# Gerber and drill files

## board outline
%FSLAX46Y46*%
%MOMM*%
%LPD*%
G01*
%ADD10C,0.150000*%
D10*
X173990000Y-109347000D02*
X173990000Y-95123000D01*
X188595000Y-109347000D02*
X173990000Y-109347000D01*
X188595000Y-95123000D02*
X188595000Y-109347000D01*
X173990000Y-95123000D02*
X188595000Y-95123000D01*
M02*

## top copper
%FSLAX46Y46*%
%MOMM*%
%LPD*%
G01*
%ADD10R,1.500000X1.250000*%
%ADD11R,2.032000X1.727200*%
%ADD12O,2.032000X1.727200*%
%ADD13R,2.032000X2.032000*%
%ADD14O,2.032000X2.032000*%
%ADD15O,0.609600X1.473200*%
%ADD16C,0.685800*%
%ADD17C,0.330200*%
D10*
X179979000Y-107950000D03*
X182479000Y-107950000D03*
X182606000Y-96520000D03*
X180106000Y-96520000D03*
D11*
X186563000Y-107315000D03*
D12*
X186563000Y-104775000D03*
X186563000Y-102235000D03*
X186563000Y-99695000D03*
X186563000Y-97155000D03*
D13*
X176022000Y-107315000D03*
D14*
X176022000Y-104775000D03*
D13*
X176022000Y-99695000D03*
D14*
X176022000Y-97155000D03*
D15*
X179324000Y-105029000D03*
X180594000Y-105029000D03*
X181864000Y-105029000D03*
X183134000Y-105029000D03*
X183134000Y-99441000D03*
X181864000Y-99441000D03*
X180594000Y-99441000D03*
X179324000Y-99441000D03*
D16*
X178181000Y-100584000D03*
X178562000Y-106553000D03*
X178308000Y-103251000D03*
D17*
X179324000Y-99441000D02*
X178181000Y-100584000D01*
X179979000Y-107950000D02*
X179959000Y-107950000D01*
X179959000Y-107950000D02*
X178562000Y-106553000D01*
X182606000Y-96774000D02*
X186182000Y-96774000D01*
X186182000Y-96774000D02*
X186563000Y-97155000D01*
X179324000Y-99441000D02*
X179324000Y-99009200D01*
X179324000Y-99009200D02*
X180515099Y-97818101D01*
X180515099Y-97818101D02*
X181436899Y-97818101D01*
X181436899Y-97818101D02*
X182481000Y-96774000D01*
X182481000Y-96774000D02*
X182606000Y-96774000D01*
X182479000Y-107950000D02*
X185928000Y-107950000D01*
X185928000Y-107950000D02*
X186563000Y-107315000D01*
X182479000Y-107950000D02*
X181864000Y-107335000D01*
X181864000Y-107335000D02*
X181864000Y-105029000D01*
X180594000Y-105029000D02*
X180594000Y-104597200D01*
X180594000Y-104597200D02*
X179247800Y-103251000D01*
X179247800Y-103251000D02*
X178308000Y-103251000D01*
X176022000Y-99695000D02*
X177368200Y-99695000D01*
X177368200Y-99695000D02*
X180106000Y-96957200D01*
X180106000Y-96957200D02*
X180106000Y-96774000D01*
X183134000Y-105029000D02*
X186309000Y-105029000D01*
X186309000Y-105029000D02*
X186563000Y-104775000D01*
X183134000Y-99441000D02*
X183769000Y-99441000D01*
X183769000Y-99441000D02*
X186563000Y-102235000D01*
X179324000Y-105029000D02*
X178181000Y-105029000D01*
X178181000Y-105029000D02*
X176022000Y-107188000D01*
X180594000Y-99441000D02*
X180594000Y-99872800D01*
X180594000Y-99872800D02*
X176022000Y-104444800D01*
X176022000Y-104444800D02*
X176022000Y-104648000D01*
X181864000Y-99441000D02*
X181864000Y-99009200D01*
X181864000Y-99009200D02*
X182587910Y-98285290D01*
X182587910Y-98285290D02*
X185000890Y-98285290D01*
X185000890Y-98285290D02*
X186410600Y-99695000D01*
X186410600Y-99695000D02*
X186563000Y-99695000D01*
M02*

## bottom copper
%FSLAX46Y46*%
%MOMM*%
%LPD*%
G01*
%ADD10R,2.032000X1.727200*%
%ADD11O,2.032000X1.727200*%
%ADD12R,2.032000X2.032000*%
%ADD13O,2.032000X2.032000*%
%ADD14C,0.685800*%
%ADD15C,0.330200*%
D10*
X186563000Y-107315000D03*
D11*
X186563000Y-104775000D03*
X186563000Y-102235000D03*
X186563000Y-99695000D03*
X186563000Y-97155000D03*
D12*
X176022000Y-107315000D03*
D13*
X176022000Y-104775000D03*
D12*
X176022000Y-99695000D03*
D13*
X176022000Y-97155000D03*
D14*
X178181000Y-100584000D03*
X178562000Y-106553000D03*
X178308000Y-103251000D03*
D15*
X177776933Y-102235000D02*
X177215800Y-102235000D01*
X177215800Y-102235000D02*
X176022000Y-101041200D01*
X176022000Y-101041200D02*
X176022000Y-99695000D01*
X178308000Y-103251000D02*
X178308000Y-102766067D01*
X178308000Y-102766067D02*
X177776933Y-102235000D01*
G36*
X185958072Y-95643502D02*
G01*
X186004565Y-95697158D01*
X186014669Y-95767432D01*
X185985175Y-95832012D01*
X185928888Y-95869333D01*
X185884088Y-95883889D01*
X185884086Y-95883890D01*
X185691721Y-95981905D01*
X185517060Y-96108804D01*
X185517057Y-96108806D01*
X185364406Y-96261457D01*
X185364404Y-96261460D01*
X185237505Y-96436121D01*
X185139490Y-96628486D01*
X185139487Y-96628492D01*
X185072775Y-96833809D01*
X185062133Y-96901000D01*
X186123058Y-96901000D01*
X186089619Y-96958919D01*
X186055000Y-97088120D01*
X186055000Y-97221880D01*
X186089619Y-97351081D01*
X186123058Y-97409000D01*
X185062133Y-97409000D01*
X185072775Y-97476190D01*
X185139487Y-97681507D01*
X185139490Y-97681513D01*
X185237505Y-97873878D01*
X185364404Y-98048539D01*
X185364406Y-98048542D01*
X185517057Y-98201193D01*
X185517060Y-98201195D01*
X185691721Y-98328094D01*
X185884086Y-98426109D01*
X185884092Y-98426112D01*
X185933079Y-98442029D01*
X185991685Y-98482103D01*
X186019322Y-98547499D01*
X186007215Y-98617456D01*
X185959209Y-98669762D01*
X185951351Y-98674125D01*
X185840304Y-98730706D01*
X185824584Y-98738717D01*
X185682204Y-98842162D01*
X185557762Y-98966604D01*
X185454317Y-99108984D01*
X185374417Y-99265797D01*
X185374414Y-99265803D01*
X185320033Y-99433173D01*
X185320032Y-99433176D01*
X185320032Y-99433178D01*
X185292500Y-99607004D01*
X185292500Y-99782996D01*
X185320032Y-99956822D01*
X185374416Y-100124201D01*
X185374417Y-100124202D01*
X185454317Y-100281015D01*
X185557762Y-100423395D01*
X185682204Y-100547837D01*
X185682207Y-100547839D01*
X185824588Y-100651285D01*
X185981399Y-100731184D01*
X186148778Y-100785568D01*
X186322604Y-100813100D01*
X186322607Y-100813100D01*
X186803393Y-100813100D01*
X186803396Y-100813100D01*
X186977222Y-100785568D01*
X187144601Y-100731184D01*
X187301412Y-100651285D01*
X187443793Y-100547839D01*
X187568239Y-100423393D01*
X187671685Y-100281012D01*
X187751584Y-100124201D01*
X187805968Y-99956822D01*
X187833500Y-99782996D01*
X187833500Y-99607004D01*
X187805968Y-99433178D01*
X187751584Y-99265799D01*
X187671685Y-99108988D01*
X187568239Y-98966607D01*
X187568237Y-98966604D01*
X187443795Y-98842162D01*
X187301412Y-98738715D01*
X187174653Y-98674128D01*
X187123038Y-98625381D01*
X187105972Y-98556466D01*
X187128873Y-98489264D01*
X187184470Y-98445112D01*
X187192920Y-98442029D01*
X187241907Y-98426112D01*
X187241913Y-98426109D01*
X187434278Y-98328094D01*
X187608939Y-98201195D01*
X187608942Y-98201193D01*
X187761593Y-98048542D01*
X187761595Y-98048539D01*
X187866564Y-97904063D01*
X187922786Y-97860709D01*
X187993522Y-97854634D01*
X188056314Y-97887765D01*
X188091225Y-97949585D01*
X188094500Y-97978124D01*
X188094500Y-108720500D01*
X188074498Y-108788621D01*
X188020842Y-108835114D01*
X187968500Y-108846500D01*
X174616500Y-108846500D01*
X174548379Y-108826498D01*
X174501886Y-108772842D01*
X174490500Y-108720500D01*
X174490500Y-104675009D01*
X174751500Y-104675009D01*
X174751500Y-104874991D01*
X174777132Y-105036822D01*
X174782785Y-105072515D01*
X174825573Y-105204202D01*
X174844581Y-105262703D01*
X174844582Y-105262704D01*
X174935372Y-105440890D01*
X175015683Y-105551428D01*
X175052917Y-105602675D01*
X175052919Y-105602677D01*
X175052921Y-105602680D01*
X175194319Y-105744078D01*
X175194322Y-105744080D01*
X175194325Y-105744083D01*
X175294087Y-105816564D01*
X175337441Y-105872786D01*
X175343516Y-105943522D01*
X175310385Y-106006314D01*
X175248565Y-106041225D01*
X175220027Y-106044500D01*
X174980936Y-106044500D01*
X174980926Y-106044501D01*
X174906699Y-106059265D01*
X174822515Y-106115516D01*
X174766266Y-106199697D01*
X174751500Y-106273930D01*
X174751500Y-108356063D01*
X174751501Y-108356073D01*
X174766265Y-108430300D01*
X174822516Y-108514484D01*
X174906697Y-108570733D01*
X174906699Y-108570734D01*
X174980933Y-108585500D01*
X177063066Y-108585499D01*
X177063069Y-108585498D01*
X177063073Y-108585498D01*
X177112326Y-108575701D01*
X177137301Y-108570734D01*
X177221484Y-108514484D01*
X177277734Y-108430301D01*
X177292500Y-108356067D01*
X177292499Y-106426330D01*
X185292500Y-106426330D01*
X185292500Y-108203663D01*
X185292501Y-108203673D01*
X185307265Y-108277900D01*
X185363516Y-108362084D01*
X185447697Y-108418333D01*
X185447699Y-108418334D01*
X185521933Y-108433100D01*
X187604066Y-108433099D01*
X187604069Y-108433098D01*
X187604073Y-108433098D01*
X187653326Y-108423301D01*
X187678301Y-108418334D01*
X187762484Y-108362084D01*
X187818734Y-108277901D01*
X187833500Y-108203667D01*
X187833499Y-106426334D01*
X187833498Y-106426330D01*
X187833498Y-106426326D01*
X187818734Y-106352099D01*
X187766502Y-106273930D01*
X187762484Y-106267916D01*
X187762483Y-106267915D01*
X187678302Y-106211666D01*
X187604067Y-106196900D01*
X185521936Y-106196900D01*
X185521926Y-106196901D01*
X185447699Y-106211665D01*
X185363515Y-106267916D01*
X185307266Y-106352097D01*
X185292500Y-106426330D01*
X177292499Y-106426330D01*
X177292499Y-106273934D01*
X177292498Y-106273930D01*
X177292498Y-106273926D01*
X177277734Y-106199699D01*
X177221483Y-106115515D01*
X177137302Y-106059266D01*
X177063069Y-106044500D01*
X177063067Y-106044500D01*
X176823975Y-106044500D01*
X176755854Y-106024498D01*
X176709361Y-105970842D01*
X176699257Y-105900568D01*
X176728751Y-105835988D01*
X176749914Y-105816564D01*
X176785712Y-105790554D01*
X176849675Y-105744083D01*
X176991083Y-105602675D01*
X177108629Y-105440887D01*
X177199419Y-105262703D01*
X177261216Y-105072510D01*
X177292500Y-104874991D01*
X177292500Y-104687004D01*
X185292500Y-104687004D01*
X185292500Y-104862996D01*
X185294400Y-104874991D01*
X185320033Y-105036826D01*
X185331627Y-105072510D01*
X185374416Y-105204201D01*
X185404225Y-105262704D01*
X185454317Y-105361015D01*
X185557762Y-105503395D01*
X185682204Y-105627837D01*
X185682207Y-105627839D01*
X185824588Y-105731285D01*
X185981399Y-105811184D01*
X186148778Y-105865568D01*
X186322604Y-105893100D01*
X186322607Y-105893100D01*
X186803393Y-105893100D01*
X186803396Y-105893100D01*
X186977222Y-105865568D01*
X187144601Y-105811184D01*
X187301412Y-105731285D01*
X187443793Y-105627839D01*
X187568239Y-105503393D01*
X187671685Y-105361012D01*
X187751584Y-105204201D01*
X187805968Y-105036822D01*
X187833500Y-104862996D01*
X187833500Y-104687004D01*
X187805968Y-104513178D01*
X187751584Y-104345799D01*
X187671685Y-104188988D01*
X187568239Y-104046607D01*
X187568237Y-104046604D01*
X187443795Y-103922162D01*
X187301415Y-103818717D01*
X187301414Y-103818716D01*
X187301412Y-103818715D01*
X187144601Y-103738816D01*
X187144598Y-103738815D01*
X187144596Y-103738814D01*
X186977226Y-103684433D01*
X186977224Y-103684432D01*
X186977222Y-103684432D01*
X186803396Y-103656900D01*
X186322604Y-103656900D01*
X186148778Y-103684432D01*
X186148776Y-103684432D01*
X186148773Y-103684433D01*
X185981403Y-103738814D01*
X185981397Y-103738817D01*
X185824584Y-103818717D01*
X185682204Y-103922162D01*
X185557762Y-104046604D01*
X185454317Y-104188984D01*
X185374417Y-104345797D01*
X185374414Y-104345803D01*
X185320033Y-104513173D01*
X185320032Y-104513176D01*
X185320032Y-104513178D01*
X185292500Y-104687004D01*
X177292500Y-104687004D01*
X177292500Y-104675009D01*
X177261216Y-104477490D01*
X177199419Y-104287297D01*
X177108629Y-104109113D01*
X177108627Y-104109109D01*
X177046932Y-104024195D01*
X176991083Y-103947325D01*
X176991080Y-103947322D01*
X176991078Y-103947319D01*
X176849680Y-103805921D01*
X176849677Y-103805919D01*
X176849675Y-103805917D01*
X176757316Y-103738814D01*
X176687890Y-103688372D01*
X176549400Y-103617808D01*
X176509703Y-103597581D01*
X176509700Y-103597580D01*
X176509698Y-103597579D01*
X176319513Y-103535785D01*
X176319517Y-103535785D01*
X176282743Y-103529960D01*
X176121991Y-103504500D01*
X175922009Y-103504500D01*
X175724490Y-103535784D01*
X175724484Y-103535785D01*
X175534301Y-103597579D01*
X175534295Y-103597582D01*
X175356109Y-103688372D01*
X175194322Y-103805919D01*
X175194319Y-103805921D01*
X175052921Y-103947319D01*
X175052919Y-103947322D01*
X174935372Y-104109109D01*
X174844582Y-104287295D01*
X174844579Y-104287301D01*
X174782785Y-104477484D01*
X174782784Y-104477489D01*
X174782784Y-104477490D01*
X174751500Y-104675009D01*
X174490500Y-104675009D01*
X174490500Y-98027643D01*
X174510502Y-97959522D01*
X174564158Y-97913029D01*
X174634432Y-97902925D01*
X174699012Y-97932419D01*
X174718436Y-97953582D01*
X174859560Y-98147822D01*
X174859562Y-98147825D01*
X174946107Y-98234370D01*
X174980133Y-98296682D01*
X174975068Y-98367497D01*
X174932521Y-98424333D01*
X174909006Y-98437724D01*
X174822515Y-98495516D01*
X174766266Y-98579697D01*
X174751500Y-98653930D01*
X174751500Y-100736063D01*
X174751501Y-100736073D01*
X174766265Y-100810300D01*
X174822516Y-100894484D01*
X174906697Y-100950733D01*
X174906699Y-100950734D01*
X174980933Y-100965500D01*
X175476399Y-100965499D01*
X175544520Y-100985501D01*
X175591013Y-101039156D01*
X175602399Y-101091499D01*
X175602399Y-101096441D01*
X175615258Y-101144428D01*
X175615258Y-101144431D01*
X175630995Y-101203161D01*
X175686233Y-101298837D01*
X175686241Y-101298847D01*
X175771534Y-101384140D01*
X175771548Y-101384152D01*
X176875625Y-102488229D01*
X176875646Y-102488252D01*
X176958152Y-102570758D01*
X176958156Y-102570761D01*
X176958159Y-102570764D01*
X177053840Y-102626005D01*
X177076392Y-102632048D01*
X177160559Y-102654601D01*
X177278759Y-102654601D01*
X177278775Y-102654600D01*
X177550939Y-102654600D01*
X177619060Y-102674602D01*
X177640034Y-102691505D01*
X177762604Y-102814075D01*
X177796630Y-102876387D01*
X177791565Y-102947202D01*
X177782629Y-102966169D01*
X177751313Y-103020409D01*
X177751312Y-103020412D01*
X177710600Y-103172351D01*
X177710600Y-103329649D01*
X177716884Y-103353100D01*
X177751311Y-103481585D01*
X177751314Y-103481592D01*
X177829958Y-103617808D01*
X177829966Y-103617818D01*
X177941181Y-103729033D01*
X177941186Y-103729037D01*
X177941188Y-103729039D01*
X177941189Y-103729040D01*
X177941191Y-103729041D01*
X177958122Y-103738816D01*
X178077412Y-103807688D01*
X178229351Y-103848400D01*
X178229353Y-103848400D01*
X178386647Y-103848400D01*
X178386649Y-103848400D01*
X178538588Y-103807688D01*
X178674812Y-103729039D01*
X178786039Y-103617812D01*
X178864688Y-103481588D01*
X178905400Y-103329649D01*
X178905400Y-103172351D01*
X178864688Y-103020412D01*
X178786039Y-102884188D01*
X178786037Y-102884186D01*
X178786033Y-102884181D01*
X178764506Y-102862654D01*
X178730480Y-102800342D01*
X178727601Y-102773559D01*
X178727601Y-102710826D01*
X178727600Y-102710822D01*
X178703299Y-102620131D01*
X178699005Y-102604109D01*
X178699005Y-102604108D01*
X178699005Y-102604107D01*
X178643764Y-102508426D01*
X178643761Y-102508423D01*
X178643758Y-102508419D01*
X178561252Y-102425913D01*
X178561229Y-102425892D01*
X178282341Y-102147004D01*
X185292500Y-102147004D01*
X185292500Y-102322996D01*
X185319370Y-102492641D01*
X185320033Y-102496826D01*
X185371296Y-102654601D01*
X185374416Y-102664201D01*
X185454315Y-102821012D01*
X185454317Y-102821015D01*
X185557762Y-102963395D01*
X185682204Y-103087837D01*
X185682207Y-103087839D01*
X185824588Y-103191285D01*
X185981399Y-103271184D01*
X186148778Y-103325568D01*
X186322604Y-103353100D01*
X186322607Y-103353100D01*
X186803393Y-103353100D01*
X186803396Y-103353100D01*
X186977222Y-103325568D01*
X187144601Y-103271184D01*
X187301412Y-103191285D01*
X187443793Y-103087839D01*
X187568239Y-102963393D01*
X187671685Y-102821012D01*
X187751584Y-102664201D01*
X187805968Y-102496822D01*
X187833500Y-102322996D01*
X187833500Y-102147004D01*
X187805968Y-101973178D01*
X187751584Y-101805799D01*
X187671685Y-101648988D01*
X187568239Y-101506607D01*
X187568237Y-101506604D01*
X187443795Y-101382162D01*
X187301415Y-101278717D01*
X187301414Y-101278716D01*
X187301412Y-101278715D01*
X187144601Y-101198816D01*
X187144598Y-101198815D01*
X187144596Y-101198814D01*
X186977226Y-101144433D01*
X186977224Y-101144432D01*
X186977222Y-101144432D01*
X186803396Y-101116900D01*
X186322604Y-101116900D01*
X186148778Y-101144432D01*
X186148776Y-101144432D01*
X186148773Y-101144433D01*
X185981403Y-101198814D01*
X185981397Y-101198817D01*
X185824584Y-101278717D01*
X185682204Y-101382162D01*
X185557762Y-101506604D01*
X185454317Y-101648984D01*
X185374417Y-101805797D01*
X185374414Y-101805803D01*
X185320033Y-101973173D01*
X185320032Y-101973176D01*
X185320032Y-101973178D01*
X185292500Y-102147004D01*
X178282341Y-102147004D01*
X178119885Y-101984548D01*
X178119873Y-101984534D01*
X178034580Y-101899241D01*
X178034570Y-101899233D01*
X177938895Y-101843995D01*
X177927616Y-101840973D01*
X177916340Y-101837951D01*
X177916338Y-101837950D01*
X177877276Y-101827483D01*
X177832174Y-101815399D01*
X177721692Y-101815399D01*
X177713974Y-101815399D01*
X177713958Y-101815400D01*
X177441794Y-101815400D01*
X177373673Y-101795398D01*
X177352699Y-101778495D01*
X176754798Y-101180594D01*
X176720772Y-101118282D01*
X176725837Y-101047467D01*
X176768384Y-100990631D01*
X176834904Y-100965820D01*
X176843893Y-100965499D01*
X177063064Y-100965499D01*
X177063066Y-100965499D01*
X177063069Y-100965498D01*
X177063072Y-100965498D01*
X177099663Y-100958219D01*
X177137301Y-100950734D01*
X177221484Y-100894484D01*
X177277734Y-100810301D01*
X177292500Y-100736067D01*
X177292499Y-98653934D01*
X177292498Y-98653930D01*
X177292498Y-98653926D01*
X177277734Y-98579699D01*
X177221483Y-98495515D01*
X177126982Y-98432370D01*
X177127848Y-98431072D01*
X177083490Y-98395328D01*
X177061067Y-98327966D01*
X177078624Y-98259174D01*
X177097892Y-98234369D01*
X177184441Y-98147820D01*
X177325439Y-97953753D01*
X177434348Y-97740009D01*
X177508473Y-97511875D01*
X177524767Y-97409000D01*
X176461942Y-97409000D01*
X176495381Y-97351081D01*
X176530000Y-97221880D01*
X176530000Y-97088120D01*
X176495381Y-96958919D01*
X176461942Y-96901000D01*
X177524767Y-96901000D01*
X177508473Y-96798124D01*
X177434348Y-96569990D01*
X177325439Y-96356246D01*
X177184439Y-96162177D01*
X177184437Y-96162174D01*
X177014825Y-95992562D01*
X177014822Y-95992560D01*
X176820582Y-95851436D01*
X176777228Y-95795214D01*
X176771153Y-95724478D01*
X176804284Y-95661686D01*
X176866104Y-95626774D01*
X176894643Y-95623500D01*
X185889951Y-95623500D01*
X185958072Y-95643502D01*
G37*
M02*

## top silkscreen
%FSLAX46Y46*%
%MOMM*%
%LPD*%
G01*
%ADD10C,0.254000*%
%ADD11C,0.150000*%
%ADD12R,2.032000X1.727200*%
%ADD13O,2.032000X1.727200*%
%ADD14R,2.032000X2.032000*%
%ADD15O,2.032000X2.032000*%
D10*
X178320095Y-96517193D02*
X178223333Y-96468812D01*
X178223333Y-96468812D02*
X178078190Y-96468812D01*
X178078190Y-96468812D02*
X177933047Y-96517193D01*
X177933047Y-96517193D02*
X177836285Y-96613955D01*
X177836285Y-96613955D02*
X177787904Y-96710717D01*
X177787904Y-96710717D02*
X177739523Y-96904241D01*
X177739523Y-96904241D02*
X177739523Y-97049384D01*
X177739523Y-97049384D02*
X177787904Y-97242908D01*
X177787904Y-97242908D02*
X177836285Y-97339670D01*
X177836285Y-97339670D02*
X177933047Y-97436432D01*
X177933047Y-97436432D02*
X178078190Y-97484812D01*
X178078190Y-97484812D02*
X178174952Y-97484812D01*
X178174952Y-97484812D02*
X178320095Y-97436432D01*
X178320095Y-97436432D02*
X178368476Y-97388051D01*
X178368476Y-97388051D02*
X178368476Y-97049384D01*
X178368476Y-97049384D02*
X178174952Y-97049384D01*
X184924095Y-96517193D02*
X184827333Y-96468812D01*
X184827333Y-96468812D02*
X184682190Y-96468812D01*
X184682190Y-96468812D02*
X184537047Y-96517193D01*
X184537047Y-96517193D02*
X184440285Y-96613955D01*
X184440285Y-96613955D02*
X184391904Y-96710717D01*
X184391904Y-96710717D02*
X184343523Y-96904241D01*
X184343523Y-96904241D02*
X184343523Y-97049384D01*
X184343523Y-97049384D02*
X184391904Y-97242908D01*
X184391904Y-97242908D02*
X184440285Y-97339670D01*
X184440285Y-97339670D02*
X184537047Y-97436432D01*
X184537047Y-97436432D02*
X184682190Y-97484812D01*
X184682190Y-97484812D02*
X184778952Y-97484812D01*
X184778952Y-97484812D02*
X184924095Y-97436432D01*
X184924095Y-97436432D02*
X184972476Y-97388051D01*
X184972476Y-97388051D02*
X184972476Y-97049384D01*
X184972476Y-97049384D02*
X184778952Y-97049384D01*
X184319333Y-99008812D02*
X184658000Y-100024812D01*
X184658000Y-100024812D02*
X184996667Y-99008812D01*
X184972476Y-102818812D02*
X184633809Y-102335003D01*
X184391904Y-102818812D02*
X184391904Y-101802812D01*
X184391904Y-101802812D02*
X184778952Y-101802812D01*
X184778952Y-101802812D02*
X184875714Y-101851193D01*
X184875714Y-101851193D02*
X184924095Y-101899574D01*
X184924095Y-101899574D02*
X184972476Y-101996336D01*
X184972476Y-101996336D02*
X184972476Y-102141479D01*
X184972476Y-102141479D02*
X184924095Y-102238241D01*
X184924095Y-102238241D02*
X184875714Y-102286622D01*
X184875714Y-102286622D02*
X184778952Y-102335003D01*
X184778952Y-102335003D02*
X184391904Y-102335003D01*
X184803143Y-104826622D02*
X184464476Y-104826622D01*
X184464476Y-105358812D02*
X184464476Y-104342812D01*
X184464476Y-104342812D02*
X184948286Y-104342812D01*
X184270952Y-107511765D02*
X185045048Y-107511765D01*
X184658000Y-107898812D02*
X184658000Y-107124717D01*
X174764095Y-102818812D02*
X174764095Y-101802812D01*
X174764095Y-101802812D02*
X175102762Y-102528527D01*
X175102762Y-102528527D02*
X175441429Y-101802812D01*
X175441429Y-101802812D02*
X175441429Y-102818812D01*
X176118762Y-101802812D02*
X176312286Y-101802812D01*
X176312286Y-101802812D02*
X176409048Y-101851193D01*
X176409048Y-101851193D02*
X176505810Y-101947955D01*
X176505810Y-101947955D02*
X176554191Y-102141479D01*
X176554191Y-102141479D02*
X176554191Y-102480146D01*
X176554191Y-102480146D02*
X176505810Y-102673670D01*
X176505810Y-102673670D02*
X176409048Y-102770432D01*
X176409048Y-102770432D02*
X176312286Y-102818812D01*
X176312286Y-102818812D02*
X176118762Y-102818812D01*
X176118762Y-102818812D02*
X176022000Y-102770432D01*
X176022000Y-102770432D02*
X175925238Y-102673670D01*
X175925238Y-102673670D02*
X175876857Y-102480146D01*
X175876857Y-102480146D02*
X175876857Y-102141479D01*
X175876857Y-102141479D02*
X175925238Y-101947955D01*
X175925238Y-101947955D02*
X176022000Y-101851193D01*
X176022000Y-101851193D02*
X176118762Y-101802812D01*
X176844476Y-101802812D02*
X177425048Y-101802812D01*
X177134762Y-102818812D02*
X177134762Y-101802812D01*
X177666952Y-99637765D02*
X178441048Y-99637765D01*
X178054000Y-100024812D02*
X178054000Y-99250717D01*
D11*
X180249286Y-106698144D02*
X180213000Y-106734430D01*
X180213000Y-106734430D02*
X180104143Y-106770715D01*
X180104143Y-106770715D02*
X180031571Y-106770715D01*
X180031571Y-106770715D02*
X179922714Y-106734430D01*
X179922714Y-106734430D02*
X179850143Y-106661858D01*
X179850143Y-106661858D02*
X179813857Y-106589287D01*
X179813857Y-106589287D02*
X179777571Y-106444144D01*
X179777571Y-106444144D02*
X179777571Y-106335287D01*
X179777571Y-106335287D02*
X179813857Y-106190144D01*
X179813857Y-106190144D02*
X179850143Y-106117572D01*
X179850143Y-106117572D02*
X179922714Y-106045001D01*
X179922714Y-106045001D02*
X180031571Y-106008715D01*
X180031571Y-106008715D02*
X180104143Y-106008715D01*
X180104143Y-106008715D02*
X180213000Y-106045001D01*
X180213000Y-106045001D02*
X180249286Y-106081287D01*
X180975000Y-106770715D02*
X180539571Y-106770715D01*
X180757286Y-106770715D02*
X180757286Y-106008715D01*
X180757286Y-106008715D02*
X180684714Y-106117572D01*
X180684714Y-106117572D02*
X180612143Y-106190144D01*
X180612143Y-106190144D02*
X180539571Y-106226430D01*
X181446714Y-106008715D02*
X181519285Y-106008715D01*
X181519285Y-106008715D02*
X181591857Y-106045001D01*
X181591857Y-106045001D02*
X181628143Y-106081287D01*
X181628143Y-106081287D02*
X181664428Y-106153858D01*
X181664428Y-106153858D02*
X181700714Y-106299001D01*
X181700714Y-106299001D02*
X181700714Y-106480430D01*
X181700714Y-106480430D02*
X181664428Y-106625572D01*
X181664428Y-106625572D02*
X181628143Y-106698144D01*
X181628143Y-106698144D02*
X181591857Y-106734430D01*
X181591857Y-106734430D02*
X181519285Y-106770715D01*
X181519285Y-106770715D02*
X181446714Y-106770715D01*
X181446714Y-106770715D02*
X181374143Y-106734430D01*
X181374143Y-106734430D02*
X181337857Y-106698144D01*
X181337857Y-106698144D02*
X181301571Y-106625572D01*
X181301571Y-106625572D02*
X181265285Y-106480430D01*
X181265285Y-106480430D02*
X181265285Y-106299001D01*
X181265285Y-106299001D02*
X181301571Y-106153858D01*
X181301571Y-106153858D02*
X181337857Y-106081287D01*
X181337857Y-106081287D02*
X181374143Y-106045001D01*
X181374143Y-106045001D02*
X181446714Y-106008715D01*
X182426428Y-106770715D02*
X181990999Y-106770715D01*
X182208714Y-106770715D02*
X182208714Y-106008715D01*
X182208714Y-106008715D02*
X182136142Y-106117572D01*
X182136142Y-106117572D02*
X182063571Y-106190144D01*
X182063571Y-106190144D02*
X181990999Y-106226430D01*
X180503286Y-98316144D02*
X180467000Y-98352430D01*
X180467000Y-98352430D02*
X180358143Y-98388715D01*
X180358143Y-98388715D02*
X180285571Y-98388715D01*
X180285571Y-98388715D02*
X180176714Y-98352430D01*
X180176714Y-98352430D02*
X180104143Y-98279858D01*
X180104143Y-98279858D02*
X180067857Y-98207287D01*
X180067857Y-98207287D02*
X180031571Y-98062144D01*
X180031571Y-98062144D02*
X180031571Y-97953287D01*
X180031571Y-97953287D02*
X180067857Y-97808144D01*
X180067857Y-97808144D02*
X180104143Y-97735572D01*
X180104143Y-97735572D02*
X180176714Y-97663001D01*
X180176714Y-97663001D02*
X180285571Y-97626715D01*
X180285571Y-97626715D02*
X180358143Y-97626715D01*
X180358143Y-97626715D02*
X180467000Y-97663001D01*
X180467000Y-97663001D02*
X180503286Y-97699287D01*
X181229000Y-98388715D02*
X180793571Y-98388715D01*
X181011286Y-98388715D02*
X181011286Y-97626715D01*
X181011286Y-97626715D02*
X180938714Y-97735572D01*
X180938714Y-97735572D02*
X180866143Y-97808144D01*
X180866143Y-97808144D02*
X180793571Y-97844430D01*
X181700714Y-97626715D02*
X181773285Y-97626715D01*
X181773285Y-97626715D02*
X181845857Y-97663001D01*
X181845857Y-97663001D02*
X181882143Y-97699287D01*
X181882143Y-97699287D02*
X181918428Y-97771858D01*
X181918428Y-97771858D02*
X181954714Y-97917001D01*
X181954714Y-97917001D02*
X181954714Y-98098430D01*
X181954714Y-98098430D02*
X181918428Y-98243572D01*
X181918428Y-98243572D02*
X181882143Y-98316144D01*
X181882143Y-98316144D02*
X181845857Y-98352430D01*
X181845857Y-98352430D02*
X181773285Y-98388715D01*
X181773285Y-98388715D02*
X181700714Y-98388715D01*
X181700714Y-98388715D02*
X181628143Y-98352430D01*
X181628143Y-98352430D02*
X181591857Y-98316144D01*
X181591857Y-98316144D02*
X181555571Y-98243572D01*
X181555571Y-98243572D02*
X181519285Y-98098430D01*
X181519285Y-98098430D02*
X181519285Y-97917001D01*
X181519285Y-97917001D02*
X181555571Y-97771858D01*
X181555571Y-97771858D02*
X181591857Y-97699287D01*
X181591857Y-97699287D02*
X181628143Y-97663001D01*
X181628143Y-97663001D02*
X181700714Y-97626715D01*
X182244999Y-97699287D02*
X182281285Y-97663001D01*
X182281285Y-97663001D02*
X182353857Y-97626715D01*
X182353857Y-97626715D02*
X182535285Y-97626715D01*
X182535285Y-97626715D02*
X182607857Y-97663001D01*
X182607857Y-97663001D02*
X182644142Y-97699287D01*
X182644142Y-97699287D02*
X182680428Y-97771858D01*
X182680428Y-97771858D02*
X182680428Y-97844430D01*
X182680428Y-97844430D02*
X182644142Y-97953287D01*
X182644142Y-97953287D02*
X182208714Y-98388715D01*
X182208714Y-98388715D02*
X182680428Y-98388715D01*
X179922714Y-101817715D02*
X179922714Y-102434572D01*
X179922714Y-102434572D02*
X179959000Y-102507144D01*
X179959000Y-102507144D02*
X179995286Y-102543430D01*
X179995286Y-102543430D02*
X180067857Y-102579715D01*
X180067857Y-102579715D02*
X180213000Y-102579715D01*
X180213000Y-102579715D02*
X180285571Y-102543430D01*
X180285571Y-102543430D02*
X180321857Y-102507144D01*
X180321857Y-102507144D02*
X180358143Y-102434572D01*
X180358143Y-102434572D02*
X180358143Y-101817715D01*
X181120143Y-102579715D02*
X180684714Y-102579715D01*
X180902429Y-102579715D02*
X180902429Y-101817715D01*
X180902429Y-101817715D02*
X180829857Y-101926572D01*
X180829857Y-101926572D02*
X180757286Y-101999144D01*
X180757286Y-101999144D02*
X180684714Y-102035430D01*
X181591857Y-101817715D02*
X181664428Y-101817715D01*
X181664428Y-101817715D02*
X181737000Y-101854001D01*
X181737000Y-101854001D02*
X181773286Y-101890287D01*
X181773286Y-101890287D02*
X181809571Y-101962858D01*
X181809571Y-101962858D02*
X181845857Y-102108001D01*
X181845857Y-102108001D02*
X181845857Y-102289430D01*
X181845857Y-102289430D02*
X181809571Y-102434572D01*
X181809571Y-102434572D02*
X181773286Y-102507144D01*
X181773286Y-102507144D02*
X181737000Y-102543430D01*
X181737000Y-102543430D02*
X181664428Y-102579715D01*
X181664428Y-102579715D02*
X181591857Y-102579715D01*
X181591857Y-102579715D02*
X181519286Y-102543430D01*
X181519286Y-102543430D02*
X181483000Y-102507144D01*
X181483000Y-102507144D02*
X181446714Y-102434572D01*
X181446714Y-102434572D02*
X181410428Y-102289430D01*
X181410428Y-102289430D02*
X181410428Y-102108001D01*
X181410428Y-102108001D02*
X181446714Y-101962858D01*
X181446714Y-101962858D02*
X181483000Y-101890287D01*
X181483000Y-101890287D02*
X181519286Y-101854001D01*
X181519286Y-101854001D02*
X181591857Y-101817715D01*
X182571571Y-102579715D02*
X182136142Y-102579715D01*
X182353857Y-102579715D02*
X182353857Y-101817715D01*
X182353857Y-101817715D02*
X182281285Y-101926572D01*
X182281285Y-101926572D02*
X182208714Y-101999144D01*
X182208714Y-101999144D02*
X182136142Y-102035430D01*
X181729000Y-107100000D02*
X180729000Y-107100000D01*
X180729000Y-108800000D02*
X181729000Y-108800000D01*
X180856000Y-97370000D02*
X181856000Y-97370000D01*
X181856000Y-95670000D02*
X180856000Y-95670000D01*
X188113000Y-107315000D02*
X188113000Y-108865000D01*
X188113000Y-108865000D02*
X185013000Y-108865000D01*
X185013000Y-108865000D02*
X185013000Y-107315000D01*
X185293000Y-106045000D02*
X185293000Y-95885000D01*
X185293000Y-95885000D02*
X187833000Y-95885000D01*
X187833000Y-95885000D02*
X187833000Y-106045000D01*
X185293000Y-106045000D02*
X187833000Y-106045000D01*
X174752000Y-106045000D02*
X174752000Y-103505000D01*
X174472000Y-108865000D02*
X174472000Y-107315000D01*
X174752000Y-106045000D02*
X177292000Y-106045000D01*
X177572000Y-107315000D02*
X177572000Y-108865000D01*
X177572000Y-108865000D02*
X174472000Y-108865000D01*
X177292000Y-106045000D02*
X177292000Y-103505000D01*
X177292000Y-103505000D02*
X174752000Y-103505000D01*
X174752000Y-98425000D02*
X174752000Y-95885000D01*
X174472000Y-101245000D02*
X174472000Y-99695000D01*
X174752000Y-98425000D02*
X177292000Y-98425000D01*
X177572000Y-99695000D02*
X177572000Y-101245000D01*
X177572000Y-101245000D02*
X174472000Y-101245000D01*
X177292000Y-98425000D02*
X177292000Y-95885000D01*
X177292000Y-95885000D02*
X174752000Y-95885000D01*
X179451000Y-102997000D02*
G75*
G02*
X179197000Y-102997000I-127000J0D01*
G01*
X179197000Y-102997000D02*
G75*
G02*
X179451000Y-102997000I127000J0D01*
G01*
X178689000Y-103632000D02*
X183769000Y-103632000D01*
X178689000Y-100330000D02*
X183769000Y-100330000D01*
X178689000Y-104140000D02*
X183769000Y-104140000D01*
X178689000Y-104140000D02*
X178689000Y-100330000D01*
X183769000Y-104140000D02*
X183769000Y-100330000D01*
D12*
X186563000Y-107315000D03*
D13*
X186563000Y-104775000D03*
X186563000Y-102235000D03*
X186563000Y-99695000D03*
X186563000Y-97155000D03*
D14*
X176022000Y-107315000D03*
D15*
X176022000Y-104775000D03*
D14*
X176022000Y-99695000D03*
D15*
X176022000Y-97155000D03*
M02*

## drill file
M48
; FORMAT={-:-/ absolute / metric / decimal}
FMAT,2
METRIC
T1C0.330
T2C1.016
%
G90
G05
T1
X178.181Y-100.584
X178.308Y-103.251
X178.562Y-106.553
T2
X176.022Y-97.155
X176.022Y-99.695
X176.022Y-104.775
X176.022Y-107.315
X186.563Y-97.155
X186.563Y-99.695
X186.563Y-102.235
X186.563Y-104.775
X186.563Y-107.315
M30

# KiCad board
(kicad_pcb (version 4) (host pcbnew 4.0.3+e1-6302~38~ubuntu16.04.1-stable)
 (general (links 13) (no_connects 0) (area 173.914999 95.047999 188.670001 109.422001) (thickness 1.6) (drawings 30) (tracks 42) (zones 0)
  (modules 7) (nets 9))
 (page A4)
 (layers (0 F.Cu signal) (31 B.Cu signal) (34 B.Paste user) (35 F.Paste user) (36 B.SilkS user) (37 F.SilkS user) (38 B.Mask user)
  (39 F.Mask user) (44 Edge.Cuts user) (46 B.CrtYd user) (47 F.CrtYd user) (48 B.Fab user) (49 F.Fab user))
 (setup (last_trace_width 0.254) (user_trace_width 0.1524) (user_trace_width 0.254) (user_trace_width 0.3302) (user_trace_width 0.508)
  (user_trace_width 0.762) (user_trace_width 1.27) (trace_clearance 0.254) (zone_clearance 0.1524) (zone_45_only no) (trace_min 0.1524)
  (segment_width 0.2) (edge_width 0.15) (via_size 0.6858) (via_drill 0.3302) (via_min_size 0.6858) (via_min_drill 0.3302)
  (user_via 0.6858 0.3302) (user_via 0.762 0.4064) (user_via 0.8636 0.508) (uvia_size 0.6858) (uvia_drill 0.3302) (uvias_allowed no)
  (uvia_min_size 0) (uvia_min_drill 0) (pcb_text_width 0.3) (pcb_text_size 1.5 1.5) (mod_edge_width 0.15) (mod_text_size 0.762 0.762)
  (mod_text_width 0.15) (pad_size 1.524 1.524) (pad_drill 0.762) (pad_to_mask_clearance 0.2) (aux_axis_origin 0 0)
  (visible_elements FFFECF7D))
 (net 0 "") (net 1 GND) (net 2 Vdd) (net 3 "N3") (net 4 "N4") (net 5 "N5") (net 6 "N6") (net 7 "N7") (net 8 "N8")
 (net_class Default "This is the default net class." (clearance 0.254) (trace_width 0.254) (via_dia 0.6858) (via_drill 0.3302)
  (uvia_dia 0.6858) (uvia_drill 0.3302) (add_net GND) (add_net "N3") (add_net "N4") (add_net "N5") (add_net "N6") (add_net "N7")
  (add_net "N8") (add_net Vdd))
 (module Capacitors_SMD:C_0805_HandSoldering (layer F.Cu) (at 181.229 107.95)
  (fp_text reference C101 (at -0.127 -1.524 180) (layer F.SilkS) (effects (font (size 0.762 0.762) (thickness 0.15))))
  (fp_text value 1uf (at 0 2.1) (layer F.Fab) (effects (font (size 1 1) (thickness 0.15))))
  (fp_line (start 0.5 -0.85) (end -0.5 -0.85) (layer F.SilkS) (width 0.15))
  (fp_line (start -0.5 0.85) (end 0.5 0.85) (layer F.SilkS) (width 0.15))
  (pad 1 smd rect (at -1.25 0) (size 1.5 1.25) (layers F.Cu F.Paste F.Mask) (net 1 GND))
  (pad 2 smd rect (at 1.25 0) (size 1.5 1.25) (layers F.Cu F.Paste F.Mask) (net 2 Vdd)))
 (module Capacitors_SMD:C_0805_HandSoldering (layer F.Cu) (at 181.356 96.52 180)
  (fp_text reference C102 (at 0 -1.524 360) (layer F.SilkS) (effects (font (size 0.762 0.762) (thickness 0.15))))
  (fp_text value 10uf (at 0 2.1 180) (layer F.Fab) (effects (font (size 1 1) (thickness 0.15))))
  (fp_line (start 0.5 -0.85) (end -0.5 -0.85) (layer F.SilkS) (width 0.15))
  (fp_line (start -0.5 0.85) (end 0.5 0.85) (layer F.SilkS) (width 0.15))
  (pad 1 smd rect (at -1.25 0 180) (size 1.5 1.25) (layers F.Cu F.Paste F.Mask) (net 1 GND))
  (pad 2 smd rect (at 1.25 0 180) (size 1.5 1.25) (layers F.Cu F.Paste F.Mask) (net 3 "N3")))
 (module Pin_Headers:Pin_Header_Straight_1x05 (layer F.Cu) (at 186.563 107.315 180)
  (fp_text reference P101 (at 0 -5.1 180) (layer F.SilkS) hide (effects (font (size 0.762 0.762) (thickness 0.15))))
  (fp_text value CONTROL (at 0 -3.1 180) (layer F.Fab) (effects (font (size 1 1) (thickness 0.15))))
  (fp_line (start -1.55 0) (end -1.55 -1.55) (layer F.SilkS) (width 0.15))
  (fp_line (start -1.55 -1.55) (end 1.55 -1.55) (layer F.SilkS) (width 0.15))
  (fp_line (start 1.55 -1.55) (end 1.55 0) (layer F.SilkS) (width 0.15))
  (fp_line (start 1.27 1.27) (end 1.27 11.43) (layer F.SilkS) (width 0.15))
  (fp_line (start 1.27 11.43) (end -1.27 11.43) (layer F.SilkS) (width 0.15))
  (fp_line (start -1.27 11.43) (end -1.27 1.27) (layer F.SilkS) (width 0.15))
  (fp_line (start 1.27 1.27) (end -1.27 1.27) (layer F.SilkS) (width 0.15))
  (pad 1 thru_hole rect (at 0 0 180) (size 2.032 1.7272) (drill 1.016) (layers *.Cu *.Mask F.SilkS) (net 2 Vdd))
  (pad 2 thru_hole oval (at 0 2.54 180) (size 2.032 1.7272) (drill 1.016) (layers *.Cu *.Mask F.SilkS) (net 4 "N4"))
  (pad 3 thru_hole oval (at 0 5.08 180) (size 2.032 1.7272) (drill 1.016) (layers *.Cu *.Mask F.SilkS) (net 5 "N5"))
  (pad 4 thru_hole oval (at 0 7.62 180) (size 2.032 1.7272) (drill 1.016) (layers *.Cu *.Mask F.SilkS) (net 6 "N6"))
  (pad 5 thru_hole oval (at 0 10.16 180) (size 2.032 1.7272) (drill 1.016) (layers *.Cu *.Mask F.SilkS) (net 1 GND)))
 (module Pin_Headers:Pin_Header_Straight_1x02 (layer F.Cu) (at 176.022 107.315 180)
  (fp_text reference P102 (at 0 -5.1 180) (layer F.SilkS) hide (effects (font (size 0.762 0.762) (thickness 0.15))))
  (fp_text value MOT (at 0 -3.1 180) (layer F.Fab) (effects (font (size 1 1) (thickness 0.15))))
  (fp_line (start 1.27 1.27) (end 1.27 3.81) (layer F.SilkS) (width 0.15))
  (fp_line (start 1.55 -1.55) (end 1.55 0) (layer F.SilkS) (width 0.15))
  (fp_line (start 1.27 1.27) (end -1.27 1.27) (layer F.SilkS) (width 0.15))
  (fp_line (start -1.55 0) (end -1.55 -1.55) (layer F.SilkS) (width 0.15))
  (fp_line (start -1.55 -1.55) (end 1.55 -1.55) (layer F.SilkS) (width 0.15))
  (fp_line (start -1.27 1.27) (end -1.27 3.81) (layer F.SilkS) (width 0.15))
  (fp_line (start -1.27 3.81) (end 1.27 3.81) (layer F.SilkS) (width 0.15))
  (pad 1 thru_hole rect (at 0 0 180) (size 2.032 2.032) (drill 1.016) (layers *.Cu *.Mask F.SilkS) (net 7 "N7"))
  (pad 2 thru_hole oval (at 0 2.54 180) (size 2.032 2.032) (drill 1.016) (layers *.Cu *.Mask F.SilkS) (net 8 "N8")))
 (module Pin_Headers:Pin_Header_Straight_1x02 (layer F.Cu) (at 176.022 99.695 180)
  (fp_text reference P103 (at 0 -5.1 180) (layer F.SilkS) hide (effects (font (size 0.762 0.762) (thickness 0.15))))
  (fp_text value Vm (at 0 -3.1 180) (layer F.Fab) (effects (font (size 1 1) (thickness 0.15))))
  (fp_line (start 1.27 1.27) (end 1.27 3.81) (layer F.SilkS) (width 0.15))
  (fp_line (start 1.55 -1.55) (end 1.55 0) (layer F.SilkS) (width 0.15))
  (fp_line (start 1.27 1.27) (end -1.27 1.27) (layer F.SilkS) (width 0.15))
  (fp_line (start -1.55 0) (end -1.55 -1.55) (layer F.SilkS) (width 0.15))
  (fp_line (start -1.55 -1.55) (end 1.55 -1.55) (layer F.SilkS) (width 0.15))
  (fp_line (start -1.27 1.27) (end -1.27 3.81) (layer F.SilkS) (width 0.15))
  (fp_line (start -1.27 3.81) (end 1.27 3.81) (layer F.SilkS) (width 0.15))
  (pad 1 thru_hole rect (at 0 0 180) (size 2.032 2.032) (drill 1.016) (layers *.Cu *.Mask F.SilkS) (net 3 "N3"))
  (pad 2 thru_hole oval (at 0 2.54 180) (size 2.032 2.032) (drill 1.016) (layers *.Cu *.Mask F.SilkS) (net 1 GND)))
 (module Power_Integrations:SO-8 (layer F.Cu) (at 181.229 102.235)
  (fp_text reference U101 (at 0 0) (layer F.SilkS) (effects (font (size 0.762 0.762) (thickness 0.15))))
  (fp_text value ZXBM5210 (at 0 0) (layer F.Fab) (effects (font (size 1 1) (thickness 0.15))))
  (fp_circle (center -1.905 0.762) (end -1.778 0.762) (layer F.SilkS) (width 0.15))
  (fp_line (start -2.54 1.397) (end 2.54 1.397) (layer F.SilkS) (width 0.15))
  (fp_line (start -2.54 -1.905) (end 2.54 -1.905) (layer F.SilkS) (width 0.15))
  (fp_line (start -2.54 1.905) (end 2.54 1.905) (layer F.SilkS) (width 0.15))
  (fp_line (start -2.54 1.905) (end -2.54 -1.905) (layer F.SilkS) (width 0.15))
  (fp_line (start 2.54 1.905) (end 2.54 -1.905) (layer F.SilkS) (width 0.15))
  (pad 1 smd oval (at -1.905 2.794) (size 0.6096 1.4732) (layers F.Cu F.Paste F.Mask) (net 7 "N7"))
  (pad 2 smd oval (at -0.635 2.794) (size 0.6096 1.4732) (layers F.Cu F.Paste F.Mask) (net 3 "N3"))
  (pad 3 smd oval (at 0.635 2.794) (size 0.6096 1.4732) (layers F.Cu F.Paste F.Mask) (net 2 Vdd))
  (pad 4 smd oval (at 1.905 2.794) (size 0.6096 1.4732) (layers F.Cu F.Paste F.Mask) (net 4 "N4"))
  (pad 5 smd oval (at 1.905 -2.794) (size 0.6096 1.4732) (layers F.Cu F.Paste F.Mask) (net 5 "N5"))
  (pad 6 smd oval (at 0.635 -2.794) (size 0.6096 1.4732) (layers F.Cu F.Paste F.Mask) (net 6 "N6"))
  (pad 7 smd oval (at -0.635 -2.794) (size 0.6096 1.4732) (layers F.Cu F.Paste F.Mask) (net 8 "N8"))
  (pad 8 smd oval (at -1.905 -2.794) (size 0.6096 1.4732) (layers F.Cu F.Paste F.Mask) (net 1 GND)))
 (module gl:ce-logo (layer B.Cu) (at 181.356 104.14 180)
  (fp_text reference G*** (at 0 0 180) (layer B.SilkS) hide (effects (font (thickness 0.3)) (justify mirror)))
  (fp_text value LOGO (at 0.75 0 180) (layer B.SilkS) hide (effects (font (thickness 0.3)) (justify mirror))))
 (gr_line (start 173.99 109.347) (end 173.99 95.123) (layer Edge.Cuts) (width 0.15))
 (gr_line (start 188.595 109.347) (end 173.99 109.347) (layer Edge.Cuts) (width 0.15))
 (gr_line (start 188.595 95.123) (end 188.595 109.347) (layer Edge.Cuts) (width 0.15))
 (gr_line (start 173.99 95.123) (end 188.595 95.123) (layer Edge.Cuts) (width 0.15))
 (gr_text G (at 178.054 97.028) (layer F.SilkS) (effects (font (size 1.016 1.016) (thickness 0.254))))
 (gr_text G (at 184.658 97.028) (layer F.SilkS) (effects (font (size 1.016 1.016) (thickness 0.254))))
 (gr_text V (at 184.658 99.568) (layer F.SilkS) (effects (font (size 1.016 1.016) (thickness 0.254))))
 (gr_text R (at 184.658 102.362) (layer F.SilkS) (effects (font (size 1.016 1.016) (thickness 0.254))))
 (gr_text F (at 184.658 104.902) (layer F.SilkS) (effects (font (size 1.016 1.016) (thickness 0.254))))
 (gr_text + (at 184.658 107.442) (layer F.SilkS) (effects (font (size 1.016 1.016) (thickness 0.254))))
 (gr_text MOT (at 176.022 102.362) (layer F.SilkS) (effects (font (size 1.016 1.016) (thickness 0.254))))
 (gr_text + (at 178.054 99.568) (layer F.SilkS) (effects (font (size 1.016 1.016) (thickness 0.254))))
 (segment (start 179.324 99.441) (end 178.181 100.584) (width 0.3302) (layer F.Cu) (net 1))
 (via (at 178.181 100.584) (size 0.6858) (drill 0.3302) (layers F.Cu B.Cu) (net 1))
 (segment (start 179.979 107.95) (end 179.959 107.95) (width 0.3302) (layer F.Cu) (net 1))
 (segment (start 179.959 107.95) (end 178.562 106.553) (width 0.3302) (layer F.Cu) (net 1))
 (via (at 178.562 106.553) (size 0.6858) (drill 0.3302) (layers F.Cu B.Cu) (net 1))
 (segment (start 182.606 96.774) (end 186.182 96.774) (width 0.3302) (layer F.Cu) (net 1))
 (segment (start 186.182 96.774) (end 186.563 97.155) (width 0.3302) (layer F.Cu) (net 1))
 (segment (start 179.324 99.441) (end 179.324 99.0092) (width 0.3302) (layer F.Cu) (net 1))
 (segment (start 179.324 99.0092) (end 180.515099 97.818101) (width 0.3302) (layer F.Cu) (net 1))
 (segment (start 180.515099 97.818101) (end 181.436899 97.818101) (width 0.3302) (layer F.Cu) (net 1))
 (segment (start 181.436899 97.818101) (end 182.481 96.774) (width 0.3302) (layer F.Cu) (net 1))
 (segment (start 182.481 96.774) (end 182.606 96.774) (width 0.3302) (layer F.Cu) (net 1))
 (segment (start 182.479 107.95) (end 185.928 107.95) (width 0.3302) (layer F.Cu) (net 2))
 (segment (start 185.928 107.95) (end 186.563 107.315) (width 0.3302) (layer F.Cu) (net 2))
 (segment (start 182.479 107.95) (end 181.864 107.335) (width 0.3302) (layer F.Cu) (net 2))
 (segment (start 181.864 107.335) (end 181.864 105.029) (width 0.3302) (layer F.Cu) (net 2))
 (segment (start 177.776933 102.235) (end 177.2158 102.235) (width 0.3302) (layer B.Cu) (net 3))
 (segment (start 177.2158 102.235) (end 176.022 101.0412) (width 0.3302) (layer B.Cu) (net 3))
 (segment (start 176.022 101.0412) (end 176.022 99.695) (width 0.3302) (layer B.Cu) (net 3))
 (segment (start 178.308 103.251) (end 178.308 102.766067) (width 0.3302) (layer B.Cu) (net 3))
 (segment (start 178.308 102.766067) (end 177.776933 102.235) (width 0.3302) (layer B.Cu) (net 3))
 (segment (start 180.594 105.029) (end 180.594 104.5972) (width 0.3302) (layer F.Cu) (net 3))
 (segment (start 180.594 104.5972) (end 179.2478 103.251) (width 0.3302) (layer F.Cu) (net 3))
 (segment (start 179.2478 103.251) (end 178.308 103.251) (width 0.3302) (layer F.Cu) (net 3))
 (via (at 178.308 103.251) (size 0.6858) (drill 0.3302) (layers F.Cu B.Cu) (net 3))
 (segment (start 176.022 99.695) (end 177.3682 99.695) (width 0.3302) (layer F.Cu) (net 3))
 (segment (start 177.3682 99.695) (end 180.106 96.9572) (width 0.3302) (layer F.Cu) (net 3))
 (segment (start 180.106 96.9572) (end 180.106 96.774) (width 0.3302) (layer F.Cu) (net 3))
 (segment (start 183.134 105.029) (end 186.309 105.029) (width 0.3302) (layer F.Cu) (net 4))
 (segment (start 186.309 105.029) (end 186.563 104.775) (width 0.3302) (layer F.Cu) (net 4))
 (segment (start 183.134 99.441) (end 183.769 99.441) (width 0.3302) (layer F.Cu) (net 5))
 (segment (start 183.769 99.441) (end 186.563 102.235) (width 0.3302) (layer F.Cu) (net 5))
 (segment (start 179.324 105.029) (end 178.181 105.029) (width 0.3302) (layer F.Cu) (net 7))
 (segment (start 178.181 105.029) (end 176.022 107.188) (width 0.3302) (layer F.Cu) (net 7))
 (segment (start 180.594 99.441) (end 180.594 99.8728) (width 0.3302) (layer F.Cu) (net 8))
 (segment (start 180.594 99.8728) (end 176.022 104.4448) (width 0.3302) (layer F.Cu) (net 8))
 (segment (start 176.022 104.4448) (end 176.022 104.648) (width 0.3302) (layer F.Cu) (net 8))
 (segment (start 181.864 99.441) (end 181.864 99.0092) (width 0.3302) (layer F.Cu) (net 6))
 (segment (start 181.864 99.0092) (end 182.58791 98.28529) (width 0.3302) (layer F.Cu) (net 6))
 (segment (start 182.58791 98.28529) (end 185.00089 98.28529) (width 0.3302) (layer F.Cu) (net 6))
 (segment (start 185.00089 98.28529) (end 186.4106 99.695) (width 0.3302) (layer F.Cu) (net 6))
 (segment (start 186.4106 99.695) (end 186.563 99.695) (width 0.3302) (layer F.Cu) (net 6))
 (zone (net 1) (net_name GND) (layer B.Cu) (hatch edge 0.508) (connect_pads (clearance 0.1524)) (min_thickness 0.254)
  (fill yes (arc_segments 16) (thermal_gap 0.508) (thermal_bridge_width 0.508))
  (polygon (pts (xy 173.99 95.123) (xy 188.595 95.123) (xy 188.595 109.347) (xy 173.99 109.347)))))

